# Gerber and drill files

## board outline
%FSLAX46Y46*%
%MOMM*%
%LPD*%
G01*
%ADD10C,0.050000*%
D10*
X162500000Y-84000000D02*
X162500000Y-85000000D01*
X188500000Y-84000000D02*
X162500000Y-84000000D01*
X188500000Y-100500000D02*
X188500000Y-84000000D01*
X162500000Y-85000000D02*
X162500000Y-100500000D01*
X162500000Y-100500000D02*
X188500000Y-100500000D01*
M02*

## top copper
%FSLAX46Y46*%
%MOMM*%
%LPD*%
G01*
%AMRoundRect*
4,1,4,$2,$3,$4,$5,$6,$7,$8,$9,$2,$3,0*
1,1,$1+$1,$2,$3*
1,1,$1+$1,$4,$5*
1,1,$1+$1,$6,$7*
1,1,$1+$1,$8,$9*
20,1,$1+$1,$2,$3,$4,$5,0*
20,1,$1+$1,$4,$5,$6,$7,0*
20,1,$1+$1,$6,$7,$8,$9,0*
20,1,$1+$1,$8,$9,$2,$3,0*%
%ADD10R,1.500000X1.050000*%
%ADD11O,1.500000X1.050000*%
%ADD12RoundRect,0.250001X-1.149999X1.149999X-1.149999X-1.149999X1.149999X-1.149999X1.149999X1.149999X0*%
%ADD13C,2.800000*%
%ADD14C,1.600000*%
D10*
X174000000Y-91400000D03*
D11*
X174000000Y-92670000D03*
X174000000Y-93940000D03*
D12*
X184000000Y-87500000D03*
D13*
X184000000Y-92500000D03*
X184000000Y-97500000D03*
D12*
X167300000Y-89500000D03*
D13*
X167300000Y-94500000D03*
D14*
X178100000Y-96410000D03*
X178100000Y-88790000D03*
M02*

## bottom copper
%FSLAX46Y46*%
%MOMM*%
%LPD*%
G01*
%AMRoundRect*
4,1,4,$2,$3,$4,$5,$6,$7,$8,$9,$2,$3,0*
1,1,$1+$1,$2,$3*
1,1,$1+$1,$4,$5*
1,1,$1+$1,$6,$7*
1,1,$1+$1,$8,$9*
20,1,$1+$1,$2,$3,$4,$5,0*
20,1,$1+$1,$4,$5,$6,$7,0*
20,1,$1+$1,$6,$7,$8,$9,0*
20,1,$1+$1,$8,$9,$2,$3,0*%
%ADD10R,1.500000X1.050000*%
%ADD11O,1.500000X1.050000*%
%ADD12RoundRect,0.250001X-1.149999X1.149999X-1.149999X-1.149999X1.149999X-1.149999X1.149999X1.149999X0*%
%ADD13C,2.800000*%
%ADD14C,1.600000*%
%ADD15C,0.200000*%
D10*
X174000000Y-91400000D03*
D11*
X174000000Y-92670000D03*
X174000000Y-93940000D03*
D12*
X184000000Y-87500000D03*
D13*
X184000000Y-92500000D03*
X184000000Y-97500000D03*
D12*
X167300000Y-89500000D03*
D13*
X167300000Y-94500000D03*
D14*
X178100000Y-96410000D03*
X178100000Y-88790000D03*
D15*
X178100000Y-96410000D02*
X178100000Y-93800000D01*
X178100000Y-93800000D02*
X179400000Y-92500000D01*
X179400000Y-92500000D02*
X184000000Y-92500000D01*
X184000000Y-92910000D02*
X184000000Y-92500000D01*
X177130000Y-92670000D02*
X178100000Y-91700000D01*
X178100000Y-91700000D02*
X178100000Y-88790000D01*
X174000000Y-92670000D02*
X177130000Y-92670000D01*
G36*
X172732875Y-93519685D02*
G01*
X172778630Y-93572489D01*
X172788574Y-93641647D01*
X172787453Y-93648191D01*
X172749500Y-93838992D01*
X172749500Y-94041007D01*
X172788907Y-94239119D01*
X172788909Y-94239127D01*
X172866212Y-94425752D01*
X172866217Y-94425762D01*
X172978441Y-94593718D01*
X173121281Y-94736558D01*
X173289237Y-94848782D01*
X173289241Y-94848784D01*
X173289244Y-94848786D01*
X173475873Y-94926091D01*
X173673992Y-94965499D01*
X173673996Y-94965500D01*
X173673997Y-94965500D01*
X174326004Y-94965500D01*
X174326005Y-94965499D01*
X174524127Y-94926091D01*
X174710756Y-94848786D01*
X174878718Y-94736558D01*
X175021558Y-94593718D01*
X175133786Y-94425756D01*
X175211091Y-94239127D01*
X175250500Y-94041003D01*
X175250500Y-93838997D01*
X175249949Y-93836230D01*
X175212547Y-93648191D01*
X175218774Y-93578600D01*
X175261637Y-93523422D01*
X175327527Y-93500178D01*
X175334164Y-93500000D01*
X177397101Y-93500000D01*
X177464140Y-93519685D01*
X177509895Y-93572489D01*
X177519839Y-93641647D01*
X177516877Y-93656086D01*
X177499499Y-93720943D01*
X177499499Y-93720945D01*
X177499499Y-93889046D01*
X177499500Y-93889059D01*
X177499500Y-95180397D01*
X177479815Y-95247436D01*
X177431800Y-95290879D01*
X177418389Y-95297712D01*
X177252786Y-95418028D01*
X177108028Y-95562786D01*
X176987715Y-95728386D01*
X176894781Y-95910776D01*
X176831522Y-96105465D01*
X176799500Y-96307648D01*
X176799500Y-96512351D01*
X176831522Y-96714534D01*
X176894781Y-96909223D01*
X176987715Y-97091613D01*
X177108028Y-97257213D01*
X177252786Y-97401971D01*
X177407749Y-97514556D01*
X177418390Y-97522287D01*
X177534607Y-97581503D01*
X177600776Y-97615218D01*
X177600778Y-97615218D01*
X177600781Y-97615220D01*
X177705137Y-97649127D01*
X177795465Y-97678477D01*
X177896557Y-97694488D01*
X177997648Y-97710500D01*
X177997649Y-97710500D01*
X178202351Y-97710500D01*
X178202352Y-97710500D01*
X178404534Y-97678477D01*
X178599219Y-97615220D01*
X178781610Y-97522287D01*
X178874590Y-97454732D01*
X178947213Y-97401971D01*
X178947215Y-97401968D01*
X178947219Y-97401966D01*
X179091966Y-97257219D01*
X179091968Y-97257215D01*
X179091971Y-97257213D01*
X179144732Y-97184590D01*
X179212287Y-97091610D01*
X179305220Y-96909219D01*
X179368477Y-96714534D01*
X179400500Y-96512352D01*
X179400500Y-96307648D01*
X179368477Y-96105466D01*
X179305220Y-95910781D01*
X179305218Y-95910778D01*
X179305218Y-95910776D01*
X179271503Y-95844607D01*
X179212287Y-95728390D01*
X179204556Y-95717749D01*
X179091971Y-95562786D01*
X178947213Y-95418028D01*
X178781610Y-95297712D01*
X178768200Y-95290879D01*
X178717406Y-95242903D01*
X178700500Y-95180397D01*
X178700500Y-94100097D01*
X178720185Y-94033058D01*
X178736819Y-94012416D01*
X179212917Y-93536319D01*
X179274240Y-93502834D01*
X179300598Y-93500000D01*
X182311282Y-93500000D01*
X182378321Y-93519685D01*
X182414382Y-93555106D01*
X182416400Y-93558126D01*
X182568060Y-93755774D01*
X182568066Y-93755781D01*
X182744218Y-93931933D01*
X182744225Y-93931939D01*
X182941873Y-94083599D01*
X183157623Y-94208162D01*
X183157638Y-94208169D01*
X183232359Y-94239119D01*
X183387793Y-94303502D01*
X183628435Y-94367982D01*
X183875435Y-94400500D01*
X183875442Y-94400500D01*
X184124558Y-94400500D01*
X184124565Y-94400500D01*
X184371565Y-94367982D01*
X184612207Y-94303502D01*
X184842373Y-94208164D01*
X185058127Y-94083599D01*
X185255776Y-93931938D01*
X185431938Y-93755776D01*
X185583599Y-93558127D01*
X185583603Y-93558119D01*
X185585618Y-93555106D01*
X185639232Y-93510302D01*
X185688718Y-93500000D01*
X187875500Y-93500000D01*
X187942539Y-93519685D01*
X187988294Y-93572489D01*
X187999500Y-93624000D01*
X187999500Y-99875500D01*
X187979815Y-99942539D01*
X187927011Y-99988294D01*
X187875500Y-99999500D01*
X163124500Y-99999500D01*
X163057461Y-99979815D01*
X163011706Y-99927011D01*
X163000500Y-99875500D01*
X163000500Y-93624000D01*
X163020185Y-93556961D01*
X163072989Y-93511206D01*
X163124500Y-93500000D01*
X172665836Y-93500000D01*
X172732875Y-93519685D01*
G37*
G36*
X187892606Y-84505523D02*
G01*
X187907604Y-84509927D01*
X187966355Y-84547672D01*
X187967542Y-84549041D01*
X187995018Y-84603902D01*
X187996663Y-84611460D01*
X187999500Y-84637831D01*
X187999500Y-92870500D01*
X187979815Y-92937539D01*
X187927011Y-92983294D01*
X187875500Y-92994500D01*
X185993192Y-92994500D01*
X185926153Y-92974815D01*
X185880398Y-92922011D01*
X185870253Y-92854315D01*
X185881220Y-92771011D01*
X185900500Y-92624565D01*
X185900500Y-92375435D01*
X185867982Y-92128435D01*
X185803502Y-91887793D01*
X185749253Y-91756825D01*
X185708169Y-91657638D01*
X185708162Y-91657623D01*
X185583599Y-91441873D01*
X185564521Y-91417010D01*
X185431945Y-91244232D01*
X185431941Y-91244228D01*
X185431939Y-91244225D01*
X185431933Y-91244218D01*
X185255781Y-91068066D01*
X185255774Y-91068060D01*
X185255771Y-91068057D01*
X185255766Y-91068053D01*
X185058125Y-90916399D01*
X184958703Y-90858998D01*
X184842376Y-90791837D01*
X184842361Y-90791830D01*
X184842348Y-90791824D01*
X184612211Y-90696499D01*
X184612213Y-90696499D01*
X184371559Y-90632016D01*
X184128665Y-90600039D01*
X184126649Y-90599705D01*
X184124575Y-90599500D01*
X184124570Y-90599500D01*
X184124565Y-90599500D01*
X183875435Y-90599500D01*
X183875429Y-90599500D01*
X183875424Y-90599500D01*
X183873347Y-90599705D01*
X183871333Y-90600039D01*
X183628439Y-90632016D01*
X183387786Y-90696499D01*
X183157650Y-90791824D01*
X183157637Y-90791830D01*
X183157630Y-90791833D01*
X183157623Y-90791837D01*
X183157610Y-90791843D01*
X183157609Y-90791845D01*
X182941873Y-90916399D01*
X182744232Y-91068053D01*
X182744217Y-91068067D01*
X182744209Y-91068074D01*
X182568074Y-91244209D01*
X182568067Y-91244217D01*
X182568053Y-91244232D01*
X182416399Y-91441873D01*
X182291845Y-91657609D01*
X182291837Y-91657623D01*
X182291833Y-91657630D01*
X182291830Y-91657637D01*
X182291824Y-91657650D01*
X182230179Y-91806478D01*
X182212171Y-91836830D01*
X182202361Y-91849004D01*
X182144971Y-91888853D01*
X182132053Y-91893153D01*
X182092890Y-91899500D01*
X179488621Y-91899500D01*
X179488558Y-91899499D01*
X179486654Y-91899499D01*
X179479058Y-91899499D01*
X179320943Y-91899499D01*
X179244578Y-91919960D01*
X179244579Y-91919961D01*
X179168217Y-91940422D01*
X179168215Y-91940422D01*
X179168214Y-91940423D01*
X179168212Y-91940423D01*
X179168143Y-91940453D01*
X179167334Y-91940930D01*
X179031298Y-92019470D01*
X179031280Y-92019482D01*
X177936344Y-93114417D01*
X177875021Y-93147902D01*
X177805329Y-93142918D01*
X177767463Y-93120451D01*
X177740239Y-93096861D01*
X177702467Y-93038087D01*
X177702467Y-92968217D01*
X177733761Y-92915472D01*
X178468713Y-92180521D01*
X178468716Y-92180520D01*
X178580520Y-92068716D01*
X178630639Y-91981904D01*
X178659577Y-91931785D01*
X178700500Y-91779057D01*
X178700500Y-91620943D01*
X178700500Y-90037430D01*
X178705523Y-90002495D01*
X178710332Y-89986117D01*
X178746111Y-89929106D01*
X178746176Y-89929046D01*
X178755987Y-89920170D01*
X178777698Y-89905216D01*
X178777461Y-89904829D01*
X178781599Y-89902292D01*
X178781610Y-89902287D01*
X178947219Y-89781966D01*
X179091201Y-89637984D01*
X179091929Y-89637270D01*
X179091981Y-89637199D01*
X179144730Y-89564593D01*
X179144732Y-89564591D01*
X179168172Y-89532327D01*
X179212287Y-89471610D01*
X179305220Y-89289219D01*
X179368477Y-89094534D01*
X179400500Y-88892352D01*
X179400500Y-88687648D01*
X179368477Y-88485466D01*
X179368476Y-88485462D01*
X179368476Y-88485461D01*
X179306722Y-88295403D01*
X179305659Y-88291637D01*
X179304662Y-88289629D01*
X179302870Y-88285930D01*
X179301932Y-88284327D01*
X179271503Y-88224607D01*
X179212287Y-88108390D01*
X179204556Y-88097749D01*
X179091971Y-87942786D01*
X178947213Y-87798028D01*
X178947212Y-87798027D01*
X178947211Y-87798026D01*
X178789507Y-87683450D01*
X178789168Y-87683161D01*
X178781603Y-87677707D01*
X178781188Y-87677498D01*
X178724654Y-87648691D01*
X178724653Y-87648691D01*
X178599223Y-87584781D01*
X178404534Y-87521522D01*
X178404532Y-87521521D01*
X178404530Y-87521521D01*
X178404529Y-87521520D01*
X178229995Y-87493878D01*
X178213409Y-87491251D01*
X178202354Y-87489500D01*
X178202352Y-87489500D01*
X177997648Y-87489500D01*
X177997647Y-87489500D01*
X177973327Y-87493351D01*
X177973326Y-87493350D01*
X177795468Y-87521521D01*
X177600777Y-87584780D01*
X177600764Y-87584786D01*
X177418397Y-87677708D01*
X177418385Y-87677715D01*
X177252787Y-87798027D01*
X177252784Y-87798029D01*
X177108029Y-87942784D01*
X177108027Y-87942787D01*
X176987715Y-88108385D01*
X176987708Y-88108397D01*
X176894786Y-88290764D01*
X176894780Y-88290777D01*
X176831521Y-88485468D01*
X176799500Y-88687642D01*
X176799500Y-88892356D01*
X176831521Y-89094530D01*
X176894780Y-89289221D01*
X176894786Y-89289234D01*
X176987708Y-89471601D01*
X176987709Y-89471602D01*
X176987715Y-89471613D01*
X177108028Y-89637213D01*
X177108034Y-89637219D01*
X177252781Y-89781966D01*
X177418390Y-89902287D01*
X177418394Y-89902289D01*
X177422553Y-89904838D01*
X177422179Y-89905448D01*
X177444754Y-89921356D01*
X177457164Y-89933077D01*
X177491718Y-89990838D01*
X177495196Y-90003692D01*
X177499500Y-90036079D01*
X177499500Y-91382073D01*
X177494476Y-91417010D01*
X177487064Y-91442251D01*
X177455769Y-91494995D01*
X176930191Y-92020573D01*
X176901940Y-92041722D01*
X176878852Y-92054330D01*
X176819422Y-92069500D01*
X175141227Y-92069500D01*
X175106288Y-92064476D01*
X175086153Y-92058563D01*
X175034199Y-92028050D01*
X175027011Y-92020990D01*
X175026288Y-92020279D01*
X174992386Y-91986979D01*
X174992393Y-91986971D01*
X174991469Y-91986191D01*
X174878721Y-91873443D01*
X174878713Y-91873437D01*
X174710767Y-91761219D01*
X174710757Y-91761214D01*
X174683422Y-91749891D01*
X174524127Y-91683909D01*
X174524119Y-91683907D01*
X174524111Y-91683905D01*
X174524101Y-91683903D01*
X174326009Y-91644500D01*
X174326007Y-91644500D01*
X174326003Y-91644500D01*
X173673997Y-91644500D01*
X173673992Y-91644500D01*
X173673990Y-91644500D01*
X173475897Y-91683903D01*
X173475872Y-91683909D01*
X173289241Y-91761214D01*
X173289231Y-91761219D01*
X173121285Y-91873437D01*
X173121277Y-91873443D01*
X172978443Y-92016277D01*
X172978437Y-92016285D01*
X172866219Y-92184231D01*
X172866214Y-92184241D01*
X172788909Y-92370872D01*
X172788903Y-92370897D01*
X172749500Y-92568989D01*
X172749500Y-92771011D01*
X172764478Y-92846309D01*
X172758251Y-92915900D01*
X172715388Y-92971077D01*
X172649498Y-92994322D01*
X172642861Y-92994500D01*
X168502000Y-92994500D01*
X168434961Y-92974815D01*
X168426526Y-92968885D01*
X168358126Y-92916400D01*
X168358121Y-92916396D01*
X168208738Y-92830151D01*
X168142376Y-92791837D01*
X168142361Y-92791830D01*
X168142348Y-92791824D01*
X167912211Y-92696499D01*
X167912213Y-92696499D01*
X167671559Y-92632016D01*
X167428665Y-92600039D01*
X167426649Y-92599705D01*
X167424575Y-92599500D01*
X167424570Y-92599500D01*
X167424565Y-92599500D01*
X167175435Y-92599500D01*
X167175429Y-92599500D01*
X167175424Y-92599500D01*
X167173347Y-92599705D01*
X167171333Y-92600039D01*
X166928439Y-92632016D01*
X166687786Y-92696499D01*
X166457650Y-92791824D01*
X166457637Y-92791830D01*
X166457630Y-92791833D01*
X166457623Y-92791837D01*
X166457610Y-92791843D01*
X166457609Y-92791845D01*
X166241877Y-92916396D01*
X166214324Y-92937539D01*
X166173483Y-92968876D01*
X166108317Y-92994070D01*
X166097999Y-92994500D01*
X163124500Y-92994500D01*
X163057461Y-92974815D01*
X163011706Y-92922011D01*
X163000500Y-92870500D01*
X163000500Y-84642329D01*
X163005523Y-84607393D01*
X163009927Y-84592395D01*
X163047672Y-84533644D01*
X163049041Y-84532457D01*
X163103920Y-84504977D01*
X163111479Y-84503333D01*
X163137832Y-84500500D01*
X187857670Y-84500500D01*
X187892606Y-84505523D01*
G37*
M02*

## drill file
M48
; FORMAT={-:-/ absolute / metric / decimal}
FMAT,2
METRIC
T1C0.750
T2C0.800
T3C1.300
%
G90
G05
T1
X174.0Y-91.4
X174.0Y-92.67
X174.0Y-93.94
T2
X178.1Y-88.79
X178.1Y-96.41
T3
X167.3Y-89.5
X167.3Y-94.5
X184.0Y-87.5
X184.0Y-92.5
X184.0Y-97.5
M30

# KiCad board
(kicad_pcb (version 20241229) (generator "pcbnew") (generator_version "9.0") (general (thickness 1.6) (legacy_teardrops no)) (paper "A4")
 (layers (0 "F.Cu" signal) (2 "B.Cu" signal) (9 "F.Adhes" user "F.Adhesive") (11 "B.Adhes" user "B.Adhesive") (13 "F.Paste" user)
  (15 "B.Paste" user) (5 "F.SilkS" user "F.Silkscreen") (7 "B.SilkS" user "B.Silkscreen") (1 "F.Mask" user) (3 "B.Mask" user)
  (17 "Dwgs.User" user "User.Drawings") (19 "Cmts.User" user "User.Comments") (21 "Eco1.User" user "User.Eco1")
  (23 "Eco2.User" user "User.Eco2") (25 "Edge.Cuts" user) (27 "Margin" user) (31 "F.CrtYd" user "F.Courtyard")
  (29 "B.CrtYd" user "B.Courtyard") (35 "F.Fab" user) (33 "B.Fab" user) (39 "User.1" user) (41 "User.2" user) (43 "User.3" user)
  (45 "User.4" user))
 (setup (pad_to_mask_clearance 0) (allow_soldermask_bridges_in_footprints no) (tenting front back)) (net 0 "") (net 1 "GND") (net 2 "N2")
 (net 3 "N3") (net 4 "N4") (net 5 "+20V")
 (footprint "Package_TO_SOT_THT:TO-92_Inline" (layer "F.Cu") (at 174 91.4 -90)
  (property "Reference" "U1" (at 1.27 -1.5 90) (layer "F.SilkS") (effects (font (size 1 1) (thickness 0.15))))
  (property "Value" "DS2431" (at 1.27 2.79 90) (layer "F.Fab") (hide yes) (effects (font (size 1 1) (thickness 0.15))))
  (pad "1" thru_hole rect (at 0 0 270) (size 1.05 1.5) (drill 0.75) (layers "*.Cu" "*.Mask") (remove_unused_layers no) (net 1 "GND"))
  (pad "2" thru_hole oval (at 1.27 0 270) (size 1.05 1.5) (drill 0.75) (layers "*.Cu" "*.Mask") (remove_unused_layers no) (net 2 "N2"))
  (pad "3" thru_hole oval (at 2.54 0 270) (size 1.05 1.5) (drill 0.75) (layers "*.Cu" "*.Mask") (remove_unused_layers no) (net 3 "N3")))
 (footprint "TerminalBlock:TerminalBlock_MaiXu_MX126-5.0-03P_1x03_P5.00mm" (layer "F.Cu") (at 184 87.5 -90)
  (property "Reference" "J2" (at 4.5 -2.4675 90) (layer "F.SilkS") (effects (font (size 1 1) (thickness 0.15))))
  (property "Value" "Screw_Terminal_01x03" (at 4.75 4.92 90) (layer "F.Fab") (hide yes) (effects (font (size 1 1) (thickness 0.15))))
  (pad "1" thru_hole roundrect (at 0 0 270) (size 2.8 2.8) (drill 1.3) (layers "*.Cu" "*.Mask") (remove_unused_layers no)
   (roundrect_rratio 0.089286) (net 1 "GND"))
  (pad "2" thru_hole circle (at 5 0 270) (size 2.8 2.8) (drill 1.3) (layers "*.Cu" "*.Mask") (remove_unused_layers no) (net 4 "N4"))
  (pad "3" thru_hole circle (at 10 0 270) (size 2.8 2.8) (drill 1.3) (layers "*.Cu" "*.Mask") (remove_unused_layers no) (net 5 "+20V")))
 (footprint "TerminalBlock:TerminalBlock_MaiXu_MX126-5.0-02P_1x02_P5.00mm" (layer "F.Cu") (at 167.3 89.5 -90)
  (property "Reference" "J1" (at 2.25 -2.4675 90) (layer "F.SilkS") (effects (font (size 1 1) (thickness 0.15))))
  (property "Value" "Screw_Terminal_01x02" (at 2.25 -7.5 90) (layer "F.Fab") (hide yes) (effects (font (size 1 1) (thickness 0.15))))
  (pad "1" thru_hole roundrect (at 0 0 270) (size 2.8 2.8) (drill 1.3) (layers "*.Cu" "*.Mask") (remove_unused_layers no)
   (roundrect_rratio 0.089286) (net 1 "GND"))
  (pad "2" thru_hole circle (at 5 0 270) (size 2.8 2.8) (drill 1.3) (layers "*.Cu" "*.Mask") (remove_unused_layers no) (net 5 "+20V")))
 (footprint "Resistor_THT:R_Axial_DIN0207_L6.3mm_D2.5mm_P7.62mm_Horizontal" (layer "F.Cu") (at 178.1 96.41 90)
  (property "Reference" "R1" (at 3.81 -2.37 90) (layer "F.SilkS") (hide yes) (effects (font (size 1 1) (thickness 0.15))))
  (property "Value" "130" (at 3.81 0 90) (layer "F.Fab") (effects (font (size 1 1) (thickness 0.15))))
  (pad "1" thru_hole circle (at 0 0 90) (size 1.6 1.6) (drill 0.8) (layers "*.Cu" "*.Mask") (remove_unused_layers no) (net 4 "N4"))
  (pad "2" thru_hole circle (at 7.62 0 90) (size 1.6 1.6) (drill 0.8) (layers "*.Cu" "*.Mask") (remove_unused_layers no) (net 2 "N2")))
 (gr_line (start 162.5 84) (end 162.5 85) (stroke (width 0.05) (type default)) (layer "Edge.Cuts"))
 (gr_line (start 188.5 84) (end 162.5 84) (stroke (width 0.05) (type default)) (layer "Edge.Cuts"))
 (gr_line (start 188.5 100.5) (end 188.5 84) (stroke (width 0.05) (type default)) (layer "Edge.Cuts"))
 (gr_line (start 162.5 85) (end 162.5 100.5) (stroke (width 0.05) (type default)) (layer "Edge.Cuts"))
 (gr_line (start 162.5 100.5) (end 188.5 100.5) (stroke (width 0.05) (type default)) (layer "Edge.Cuts"))
 (segment (start 178.1 96.41) (end 178.1 93.8) (width 0.2) (layer "B.Cu") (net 4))
 (segment (start 178.1 93.8) (end 179.4 92.5) (width 0.2) (layer "B.Cu") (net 4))
 (segment (start 179.4 92.5) (end 184 92.5) (width 0.2) (layer "B.Cu") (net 4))
 (segment (start 184 92.91) (end 184 92.5) (width 0.2) (layer "B.Cu") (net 4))
 (segment (start 177.13 92.67) (end 178.1 91.7) (width 0.2) (layer "B.Cu") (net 2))
 (segment (start 178.1 91.7) (end 178.1 88.79) (width 0.2) (layer "B.Cu") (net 2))
 (segment (start 174 92.67) (end 177.13 92.67) (width 0.2) (layer "B.Cu") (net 2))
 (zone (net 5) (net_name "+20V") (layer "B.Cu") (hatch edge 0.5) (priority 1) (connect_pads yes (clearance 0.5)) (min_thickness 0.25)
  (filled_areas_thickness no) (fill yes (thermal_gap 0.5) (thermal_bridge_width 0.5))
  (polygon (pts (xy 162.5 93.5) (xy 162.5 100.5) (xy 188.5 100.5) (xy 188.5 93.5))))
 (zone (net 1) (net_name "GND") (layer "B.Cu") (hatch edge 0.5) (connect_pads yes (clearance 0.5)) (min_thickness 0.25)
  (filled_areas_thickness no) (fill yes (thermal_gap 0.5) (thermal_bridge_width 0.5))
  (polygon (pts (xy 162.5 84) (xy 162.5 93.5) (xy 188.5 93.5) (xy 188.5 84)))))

